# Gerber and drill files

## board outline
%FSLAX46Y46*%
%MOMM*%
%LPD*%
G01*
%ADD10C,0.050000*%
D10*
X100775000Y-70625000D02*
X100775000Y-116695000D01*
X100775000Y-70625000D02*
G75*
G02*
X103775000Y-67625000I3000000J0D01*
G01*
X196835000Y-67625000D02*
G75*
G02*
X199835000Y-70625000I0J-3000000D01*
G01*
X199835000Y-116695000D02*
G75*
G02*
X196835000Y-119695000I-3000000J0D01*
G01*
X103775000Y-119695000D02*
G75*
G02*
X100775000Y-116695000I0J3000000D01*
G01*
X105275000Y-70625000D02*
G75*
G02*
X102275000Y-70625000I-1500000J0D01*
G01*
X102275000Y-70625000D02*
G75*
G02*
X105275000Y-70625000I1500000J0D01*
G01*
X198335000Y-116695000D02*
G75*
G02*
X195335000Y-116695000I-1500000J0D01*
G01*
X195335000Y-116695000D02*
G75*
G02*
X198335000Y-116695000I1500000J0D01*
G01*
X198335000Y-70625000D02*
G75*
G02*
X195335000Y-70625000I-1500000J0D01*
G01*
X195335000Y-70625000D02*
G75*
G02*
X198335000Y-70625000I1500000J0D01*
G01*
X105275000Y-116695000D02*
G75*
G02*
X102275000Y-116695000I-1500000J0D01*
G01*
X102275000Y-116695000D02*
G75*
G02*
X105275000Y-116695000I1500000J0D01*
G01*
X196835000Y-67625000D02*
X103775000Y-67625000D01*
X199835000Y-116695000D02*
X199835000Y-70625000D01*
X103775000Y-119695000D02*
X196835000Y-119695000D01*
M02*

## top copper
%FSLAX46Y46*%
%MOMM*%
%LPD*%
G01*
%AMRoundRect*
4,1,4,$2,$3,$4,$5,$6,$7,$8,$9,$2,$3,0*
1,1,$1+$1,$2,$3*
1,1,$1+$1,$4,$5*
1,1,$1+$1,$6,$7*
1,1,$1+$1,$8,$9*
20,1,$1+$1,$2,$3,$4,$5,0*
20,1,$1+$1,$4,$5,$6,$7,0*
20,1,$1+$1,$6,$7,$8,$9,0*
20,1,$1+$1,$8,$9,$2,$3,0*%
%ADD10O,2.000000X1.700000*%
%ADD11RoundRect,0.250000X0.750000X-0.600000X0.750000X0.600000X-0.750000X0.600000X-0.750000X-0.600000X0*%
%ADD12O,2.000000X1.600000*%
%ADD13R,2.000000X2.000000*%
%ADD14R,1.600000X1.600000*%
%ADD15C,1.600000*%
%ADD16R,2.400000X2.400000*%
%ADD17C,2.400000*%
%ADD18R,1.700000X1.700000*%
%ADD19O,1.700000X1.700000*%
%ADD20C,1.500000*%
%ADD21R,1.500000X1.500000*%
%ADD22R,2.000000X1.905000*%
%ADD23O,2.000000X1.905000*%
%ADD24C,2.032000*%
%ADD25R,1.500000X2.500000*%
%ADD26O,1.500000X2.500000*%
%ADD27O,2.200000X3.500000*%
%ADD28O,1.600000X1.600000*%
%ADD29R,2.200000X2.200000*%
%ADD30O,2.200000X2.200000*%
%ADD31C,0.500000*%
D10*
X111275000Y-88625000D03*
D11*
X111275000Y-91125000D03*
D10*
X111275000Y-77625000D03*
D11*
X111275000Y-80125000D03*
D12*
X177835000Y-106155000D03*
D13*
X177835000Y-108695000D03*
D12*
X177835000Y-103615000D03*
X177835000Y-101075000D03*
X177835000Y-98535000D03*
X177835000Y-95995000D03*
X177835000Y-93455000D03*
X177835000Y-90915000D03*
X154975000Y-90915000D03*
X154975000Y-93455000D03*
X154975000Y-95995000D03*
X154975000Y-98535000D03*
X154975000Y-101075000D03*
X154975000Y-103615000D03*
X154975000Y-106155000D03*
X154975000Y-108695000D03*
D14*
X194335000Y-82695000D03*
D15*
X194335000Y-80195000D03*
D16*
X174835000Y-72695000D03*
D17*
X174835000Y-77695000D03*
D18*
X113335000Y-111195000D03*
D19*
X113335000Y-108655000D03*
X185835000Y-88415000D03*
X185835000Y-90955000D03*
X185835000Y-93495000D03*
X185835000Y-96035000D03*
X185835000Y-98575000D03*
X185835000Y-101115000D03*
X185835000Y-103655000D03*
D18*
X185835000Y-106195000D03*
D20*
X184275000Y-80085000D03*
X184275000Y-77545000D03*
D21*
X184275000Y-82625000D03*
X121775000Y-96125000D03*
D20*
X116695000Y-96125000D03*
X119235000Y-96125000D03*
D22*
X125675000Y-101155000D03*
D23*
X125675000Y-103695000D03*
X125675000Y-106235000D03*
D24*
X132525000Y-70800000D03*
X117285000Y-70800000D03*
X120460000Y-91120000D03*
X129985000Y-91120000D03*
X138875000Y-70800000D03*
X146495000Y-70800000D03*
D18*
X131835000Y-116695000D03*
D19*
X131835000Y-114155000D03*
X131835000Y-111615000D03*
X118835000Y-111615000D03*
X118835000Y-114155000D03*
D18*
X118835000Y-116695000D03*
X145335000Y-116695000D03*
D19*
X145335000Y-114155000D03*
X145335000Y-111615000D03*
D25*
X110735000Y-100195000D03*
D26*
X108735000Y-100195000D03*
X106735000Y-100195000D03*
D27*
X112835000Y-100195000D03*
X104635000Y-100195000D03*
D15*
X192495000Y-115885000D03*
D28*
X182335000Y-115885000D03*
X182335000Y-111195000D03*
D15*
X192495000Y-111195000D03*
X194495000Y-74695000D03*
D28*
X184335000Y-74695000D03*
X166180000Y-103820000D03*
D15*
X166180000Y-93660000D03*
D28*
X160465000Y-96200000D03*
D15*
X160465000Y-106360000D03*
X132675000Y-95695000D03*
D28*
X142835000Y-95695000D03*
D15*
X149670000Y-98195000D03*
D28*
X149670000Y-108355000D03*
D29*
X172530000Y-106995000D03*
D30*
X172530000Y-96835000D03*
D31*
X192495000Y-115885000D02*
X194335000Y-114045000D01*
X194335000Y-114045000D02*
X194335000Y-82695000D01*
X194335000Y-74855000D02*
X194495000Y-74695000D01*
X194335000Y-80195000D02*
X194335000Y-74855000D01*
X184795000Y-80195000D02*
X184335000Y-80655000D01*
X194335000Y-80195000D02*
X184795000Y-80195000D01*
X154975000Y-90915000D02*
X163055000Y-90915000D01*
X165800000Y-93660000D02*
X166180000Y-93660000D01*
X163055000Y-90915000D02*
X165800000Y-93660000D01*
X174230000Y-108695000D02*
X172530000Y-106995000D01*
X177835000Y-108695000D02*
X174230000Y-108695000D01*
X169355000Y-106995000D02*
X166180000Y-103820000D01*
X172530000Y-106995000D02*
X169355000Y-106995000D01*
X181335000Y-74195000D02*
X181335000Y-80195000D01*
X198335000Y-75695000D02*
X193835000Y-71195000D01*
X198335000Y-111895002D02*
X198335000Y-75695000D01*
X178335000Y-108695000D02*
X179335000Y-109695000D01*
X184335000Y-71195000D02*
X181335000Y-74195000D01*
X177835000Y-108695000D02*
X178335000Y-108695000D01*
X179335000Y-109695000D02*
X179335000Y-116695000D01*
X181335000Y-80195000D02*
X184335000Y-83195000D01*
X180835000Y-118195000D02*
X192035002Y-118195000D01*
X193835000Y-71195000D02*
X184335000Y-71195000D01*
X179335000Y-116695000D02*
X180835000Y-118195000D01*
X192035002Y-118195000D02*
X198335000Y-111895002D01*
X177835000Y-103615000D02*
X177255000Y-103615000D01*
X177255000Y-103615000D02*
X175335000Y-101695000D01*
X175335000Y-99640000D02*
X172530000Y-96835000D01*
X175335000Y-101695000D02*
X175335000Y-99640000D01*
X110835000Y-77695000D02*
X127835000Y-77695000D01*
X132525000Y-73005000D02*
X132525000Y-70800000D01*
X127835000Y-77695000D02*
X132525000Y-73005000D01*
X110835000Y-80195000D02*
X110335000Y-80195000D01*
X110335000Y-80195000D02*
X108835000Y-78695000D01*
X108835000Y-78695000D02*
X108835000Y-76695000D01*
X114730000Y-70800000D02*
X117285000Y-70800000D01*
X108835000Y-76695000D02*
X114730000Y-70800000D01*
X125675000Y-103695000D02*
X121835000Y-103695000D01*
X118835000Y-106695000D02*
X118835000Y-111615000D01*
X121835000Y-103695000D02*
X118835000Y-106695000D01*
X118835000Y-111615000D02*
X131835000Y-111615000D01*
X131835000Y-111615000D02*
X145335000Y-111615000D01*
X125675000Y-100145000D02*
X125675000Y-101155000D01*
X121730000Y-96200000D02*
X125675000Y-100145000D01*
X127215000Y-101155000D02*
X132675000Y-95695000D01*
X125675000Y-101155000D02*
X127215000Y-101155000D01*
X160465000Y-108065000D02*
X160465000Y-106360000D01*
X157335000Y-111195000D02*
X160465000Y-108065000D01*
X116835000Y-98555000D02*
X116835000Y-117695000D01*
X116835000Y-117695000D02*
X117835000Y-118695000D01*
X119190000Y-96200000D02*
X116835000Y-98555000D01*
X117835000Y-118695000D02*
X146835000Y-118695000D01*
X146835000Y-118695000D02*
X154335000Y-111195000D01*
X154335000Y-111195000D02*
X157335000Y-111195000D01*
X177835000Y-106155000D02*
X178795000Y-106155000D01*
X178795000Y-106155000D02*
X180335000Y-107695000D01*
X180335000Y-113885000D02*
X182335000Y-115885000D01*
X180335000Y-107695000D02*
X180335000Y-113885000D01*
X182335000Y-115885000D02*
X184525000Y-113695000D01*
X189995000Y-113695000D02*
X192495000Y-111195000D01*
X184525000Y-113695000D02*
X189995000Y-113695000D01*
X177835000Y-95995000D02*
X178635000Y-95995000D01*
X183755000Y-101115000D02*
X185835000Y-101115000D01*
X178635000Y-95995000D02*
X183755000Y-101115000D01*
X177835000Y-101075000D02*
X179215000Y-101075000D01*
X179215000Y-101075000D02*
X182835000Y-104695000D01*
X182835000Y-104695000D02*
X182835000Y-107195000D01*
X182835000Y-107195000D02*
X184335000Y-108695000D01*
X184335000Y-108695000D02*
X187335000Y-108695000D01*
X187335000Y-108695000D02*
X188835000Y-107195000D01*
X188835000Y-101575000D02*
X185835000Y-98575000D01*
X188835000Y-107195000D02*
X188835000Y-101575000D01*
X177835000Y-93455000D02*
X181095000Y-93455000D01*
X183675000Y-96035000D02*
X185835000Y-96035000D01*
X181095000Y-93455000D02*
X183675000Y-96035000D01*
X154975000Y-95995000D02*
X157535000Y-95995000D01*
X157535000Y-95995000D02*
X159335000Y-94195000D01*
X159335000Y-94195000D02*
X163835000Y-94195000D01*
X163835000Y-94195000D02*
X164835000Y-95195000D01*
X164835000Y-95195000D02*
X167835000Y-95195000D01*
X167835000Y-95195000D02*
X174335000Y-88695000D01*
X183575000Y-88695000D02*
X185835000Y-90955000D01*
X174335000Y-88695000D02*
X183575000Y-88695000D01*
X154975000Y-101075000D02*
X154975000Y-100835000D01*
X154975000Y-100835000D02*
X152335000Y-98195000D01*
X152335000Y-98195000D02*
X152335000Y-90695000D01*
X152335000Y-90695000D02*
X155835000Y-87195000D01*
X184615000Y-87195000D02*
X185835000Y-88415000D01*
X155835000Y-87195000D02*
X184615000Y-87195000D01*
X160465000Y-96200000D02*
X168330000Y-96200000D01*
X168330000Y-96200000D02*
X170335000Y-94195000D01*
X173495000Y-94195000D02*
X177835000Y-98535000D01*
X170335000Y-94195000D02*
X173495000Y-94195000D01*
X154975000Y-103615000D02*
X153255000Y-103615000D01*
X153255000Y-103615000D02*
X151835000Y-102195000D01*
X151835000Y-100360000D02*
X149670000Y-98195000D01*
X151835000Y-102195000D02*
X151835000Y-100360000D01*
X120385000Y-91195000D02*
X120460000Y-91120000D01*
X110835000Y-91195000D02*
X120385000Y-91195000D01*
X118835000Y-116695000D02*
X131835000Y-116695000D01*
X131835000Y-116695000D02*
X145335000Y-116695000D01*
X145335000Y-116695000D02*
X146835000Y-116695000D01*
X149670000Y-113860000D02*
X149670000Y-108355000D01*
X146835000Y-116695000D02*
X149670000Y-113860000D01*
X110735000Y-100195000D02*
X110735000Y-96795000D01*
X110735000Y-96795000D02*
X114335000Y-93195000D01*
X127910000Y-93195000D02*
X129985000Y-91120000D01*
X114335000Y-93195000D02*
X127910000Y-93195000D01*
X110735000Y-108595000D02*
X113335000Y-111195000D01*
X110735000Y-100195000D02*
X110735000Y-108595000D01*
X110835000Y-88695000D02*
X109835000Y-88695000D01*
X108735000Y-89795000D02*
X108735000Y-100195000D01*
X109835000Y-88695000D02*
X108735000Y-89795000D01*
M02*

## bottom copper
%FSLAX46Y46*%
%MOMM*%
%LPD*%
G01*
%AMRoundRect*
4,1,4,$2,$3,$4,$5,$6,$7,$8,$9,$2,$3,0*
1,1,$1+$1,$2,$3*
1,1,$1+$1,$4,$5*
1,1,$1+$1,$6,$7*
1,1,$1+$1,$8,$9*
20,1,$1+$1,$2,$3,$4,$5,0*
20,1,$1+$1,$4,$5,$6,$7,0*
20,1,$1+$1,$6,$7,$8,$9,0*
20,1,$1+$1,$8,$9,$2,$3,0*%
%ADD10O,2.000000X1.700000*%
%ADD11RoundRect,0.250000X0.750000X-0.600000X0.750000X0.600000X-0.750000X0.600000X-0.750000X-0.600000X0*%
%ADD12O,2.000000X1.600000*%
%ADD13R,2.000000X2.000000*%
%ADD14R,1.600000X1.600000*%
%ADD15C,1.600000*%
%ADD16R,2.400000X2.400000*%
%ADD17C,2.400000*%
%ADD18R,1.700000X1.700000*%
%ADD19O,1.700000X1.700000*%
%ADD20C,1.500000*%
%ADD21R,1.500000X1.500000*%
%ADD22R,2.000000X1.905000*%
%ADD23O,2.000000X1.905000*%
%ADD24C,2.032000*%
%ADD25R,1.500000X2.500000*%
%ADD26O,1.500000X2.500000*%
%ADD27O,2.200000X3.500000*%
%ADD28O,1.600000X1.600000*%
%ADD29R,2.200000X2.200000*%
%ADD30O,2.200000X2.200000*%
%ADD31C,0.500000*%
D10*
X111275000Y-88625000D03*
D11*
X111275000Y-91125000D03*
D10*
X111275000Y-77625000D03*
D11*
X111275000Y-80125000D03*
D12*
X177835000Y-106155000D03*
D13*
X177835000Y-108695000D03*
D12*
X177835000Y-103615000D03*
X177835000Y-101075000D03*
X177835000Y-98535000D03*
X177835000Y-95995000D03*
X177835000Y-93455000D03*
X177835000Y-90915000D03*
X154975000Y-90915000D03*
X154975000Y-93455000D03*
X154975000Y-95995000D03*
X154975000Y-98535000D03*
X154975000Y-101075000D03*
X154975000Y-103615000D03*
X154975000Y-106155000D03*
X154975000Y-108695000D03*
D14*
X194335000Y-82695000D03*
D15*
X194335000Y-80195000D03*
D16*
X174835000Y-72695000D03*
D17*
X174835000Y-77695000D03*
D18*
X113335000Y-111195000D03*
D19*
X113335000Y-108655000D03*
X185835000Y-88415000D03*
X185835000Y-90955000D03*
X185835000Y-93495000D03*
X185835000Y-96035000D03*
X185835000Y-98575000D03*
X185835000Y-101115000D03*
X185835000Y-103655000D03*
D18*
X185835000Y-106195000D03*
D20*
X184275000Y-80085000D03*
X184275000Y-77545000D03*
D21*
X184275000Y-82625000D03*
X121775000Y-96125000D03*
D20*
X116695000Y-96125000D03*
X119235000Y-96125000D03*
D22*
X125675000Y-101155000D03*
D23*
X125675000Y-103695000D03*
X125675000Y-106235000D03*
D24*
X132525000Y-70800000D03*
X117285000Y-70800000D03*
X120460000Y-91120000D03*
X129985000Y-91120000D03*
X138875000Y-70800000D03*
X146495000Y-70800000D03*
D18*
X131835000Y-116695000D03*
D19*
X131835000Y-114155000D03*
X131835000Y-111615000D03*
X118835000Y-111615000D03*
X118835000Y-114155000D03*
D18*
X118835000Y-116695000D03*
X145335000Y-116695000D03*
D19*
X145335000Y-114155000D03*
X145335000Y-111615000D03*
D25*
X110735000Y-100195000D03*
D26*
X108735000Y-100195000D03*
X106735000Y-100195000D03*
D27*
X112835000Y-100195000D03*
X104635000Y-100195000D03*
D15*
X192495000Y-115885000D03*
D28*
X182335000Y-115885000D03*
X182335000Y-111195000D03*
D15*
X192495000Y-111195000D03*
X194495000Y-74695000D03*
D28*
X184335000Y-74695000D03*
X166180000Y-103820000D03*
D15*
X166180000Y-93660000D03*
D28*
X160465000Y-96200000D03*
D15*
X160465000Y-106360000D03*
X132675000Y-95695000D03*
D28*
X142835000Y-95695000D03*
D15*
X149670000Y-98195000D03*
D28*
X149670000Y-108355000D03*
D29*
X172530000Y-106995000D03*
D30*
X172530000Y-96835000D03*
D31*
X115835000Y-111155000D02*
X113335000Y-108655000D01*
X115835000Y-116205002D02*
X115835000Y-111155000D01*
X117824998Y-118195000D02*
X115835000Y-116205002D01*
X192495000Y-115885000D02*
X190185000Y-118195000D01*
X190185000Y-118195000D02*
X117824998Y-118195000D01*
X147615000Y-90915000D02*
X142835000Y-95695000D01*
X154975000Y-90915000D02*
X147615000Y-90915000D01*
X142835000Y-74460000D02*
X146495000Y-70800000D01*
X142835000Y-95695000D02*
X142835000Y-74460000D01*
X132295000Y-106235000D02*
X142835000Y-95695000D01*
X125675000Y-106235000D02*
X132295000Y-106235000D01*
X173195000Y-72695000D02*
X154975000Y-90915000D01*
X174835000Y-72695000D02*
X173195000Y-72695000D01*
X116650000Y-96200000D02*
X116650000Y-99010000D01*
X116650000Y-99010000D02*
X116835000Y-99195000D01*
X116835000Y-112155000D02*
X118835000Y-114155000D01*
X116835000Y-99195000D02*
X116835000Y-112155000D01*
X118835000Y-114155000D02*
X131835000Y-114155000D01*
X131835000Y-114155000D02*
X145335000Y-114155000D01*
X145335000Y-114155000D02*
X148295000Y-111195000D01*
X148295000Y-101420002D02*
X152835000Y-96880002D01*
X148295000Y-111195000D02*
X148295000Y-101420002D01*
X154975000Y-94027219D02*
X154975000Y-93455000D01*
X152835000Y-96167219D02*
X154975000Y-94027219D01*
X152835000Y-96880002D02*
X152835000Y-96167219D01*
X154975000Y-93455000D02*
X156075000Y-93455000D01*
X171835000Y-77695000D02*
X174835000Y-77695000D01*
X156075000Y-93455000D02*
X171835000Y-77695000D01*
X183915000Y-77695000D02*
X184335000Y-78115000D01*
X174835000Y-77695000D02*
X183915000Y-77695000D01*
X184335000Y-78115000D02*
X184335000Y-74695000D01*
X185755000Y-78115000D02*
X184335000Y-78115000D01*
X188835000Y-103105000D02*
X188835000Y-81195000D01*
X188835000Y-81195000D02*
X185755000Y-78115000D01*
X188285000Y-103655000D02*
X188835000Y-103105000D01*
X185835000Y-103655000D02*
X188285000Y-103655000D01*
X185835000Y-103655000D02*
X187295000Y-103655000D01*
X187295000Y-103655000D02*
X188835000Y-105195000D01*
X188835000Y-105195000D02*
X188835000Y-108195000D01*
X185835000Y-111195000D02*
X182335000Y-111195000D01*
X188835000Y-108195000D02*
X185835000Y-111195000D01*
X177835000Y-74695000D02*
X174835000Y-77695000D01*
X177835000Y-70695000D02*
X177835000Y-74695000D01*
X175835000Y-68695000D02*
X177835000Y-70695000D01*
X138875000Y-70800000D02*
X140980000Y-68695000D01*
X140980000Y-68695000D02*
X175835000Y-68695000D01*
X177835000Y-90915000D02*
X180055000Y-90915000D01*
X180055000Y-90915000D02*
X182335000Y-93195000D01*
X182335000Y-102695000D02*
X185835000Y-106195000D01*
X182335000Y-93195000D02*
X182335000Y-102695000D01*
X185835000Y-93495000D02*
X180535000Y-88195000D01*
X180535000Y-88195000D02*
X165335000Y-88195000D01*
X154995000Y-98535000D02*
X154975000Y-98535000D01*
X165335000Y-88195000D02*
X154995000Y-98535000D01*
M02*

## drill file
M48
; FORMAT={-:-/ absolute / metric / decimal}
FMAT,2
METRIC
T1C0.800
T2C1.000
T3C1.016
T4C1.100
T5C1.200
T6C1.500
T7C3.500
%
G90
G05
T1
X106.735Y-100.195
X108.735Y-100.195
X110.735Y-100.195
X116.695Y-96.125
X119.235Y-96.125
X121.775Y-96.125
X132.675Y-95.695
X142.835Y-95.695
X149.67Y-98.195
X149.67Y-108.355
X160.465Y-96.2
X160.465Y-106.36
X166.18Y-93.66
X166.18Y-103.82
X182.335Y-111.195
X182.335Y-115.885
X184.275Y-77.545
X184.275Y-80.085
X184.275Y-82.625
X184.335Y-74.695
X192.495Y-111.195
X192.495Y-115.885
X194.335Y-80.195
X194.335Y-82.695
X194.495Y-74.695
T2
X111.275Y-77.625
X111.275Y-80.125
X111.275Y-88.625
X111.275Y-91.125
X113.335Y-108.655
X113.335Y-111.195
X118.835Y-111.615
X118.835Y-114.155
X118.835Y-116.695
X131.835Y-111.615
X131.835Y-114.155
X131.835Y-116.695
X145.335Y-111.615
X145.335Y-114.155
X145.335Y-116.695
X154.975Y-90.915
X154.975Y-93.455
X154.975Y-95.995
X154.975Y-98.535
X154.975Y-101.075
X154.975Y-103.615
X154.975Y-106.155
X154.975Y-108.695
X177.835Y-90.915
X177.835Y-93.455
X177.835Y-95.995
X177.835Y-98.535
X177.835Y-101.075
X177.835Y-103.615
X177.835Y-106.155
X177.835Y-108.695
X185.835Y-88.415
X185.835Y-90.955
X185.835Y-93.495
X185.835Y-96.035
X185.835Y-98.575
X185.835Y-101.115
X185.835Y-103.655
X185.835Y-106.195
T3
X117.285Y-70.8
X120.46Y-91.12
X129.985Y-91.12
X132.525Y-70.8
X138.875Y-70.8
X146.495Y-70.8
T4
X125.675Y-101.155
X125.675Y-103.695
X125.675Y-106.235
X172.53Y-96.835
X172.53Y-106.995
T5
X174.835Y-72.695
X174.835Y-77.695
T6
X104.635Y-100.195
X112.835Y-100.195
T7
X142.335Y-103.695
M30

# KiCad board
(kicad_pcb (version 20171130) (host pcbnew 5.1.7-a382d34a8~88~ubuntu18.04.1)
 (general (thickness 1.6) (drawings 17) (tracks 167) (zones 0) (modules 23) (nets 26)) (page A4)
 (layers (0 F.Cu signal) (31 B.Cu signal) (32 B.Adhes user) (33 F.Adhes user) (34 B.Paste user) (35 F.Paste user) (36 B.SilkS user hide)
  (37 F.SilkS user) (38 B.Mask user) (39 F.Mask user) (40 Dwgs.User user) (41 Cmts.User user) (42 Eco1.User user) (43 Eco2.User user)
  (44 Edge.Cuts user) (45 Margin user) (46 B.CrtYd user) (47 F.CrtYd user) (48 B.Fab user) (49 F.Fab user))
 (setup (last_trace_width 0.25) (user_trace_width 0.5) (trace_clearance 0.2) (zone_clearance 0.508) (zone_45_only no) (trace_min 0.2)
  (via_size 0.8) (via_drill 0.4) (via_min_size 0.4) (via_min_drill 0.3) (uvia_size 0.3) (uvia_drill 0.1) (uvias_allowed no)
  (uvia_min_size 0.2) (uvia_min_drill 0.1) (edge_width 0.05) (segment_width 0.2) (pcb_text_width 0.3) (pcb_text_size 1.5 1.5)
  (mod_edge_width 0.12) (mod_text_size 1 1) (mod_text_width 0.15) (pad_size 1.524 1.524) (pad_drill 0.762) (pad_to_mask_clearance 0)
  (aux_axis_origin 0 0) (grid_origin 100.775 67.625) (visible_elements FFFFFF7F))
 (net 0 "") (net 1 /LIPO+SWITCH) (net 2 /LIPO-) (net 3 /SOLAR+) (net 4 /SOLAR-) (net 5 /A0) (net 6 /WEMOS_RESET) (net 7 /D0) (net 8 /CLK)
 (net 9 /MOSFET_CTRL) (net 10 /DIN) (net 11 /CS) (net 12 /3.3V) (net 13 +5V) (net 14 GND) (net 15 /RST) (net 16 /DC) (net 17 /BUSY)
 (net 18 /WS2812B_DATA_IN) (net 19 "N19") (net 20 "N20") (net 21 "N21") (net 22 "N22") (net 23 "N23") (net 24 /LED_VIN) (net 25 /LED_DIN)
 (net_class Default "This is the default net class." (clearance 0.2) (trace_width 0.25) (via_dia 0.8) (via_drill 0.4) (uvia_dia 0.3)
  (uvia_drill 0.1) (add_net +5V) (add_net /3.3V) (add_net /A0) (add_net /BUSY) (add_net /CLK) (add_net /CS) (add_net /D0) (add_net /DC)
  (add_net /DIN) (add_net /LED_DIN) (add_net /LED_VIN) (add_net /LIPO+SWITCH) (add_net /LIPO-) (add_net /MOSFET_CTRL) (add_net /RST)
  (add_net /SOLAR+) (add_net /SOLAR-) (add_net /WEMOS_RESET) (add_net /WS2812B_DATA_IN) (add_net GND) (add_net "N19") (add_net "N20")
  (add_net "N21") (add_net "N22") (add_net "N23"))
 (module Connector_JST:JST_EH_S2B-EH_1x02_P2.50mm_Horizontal (layer F.Cu) (at 111.275 91.125 90)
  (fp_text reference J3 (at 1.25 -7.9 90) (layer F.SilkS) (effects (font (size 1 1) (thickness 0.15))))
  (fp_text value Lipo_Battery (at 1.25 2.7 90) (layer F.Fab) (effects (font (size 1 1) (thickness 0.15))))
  (pad 2 thru_hole oval (at 2.5 0 90) (size 1.7 2) (drill 1) (layers *.Cu *.Mask) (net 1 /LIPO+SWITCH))
  (pad 1 thru_hole roundrect (at 0 0 90) (size 1.7 2) (drill 1) (layers *.Cu *.Mask) (roundrect_rratio 0.147059) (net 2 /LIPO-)))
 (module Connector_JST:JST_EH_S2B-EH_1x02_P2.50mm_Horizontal (layer F.Cu) (at 111.275 80.125 90)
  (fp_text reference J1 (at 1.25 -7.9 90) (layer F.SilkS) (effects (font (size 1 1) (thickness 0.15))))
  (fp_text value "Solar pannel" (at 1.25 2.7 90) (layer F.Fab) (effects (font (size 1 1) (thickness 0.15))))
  (pad 2 thru_hole oval (at 2.5 0 90) (size 1.7 2) (drill 1) (layers *.Cu *.Mask) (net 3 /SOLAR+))
  (pad 1 thru_hole roundrect (at 0 0 90) (size 1.7 2) (drill 1) (layers *.Cu *.Mask) (roundrect_rratio 0.147059) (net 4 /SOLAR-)))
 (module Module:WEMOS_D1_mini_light (layer F.Cu) (at 177.835 108.695 180)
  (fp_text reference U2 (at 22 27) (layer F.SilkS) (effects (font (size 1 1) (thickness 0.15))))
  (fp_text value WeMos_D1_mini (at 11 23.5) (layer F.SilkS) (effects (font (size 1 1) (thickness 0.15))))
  (pad 2 thru_hole oval (at 0 2.54 180) (size 2 1.6) (drill 1) (layers *.Cu *.Mask) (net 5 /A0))
  (pad 1 thru_hole rect (at 0 0 180) (size 2 2) (drill 1) (layers *.Cu *.Mask) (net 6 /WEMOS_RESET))
  (pad 3 thru_hole oval (at 0 5.08 180) (size 2 1.6) (drill 1) (layers *.Cu *.Mask) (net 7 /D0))
  (pad 4 thru_hole oval (at 0 7.62 180) (size 2 1.6) (drill 1) (layers *.Cu *.Mask) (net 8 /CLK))
  (pad 5 thru_hole oval (at 0 10.16 180) (size 2 1.6) (drill 1) (layers *.Cu *.Mask) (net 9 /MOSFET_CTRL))
  (pad 6 thru_hole oval (at 0 12.7 180) (size 2 1.6) (drill 1) (layers *.Cu *.Mask) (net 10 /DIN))
  (pad 7 thru_hole oval (at 0 15.24 180) (size 2 1.6) (drill 1) (layers *.Cu *.Mask) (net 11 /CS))
  (pad 8 thru_hole oval (at 0 17.78 180) (size 2 1.6) (drill 1) (layers *.Cu *.Mask) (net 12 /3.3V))
  (pad 9 thru_hole oval (at 22.86 17.78 180) (size 2 1.6) (drill 1) (layers *.Cu *.Mask) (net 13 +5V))
  (pad 10 thru_hole oval (at 22.86 15.24 180) (size 2 1.6) (drill 1) (layers *.Cu *.Mask) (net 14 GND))
  (pad 11 thru_hole oval (at 22.86 12.7 180) (size 2 1.6) (drill 1) (layers *.Cu *.Mask) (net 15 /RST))
  (pad 12 thru_hole oval (at 22.86 10.16 180) (size 2 1.6) (drill 1) (layers *.Cu *.Mask) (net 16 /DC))
  (pad 13 thru_hole oval (at 22.86 7.62 180) (size 2 1.6) (drill 1) (layers *.Cu *.Mask) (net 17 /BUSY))
  (pad 14 thru_hole oval (at 22.86 5.08 180) (size 2 1.6) (drill 1) (layers *.Cu *.Mask) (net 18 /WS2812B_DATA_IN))
  (pad 15 thru_hole oval (at 22.86 2.54 180) (size 2 1.6) (drill 1) (layers *.Cu *.Mask))
  (pad 16 thru_hole oval (at 22.86 0 180) (size 2 1.6) (drill 1) (layers *.Cu *.Mask)))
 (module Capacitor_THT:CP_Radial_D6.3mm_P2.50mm (layer F.Cu) (at 194.335 82.695 90)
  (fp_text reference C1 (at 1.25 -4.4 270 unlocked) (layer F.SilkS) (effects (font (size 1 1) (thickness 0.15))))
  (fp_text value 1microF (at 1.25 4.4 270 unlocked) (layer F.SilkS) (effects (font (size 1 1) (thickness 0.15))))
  (pad 1 thru_hole rect (at 0 0 90) (size 1.6 1.6) (drill 0.8) (layers *.Cu *.Mask) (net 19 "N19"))
  (pad 2 thru_hole circle (at 2.5 0 90) (size 1.6 1.6) (drill 0.8) (layers *.Cu *.Mask) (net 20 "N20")))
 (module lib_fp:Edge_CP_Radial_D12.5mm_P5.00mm (layer F.Cu) (at 174.835 75.195 270)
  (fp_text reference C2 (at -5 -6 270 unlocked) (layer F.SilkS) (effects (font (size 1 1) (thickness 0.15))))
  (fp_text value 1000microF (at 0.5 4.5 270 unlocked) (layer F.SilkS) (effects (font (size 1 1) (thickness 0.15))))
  (pad 1 thru_hole rect (at -2.5 0 270) (size 2.4 2.4) (drill 1.2) (layers *.Cu *.Mask) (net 13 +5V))
  (pad 2 thru_hole circle (at 2.5 0 270) (size 2.4 2.4) (drill 1.2) (layers *.Cu *.Mask) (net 14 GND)))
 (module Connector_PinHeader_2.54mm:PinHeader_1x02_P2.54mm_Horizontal (layer F.Cu) (at 113.335 111.195 180)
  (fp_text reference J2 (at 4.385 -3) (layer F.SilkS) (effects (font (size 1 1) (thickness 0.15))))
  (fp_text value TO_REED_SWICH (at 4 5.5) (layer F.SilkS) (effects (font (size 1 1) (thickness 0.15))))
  (pad 1 thru_hole rect (at 0 0 180) (size 1.7 1.7) (drill 1) (layers *.Cu *.Mask) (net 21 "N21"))
  (pad 2 thru_hole oval (at 0 2.54 180) (size 1.7 1.7) (drill 1) (layers *.Cu *.Mask) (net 19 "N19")))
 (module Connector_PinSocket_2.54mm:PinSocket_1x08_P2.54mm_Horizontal (layer F.Cu) (at 185.835 106.195 180)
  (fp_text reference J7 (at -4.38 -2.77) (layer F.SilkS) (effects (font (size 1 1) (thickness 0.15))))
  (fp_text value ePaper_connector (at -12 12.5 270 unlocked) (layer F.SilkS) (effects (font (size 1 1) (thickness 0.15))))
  (pad 8 thru_hole oval (at 0 17.78 180) (size 1.7 1.7) (drill 1) (layers *.Cu *.Mask) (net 17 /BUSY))
  (pad 7 thru_hole oval (at 0 15.24 180) (size 1.7 1.7) (drill 1) (layers *.Cu *.Mask) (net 15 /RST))
  (pad 6 thru_hole oval (at 0 12.7 180) (size 1.7 1.7) (drill 1) (layers *.Cu *.Mask) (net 16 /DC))
  (pad 5 thru_hole oval (at 0 10.16 180) (size 1.7 1.7) (drill 1) (layers *.Cu *.Mask) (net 11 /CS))
  (pad 4 thru_hole oval (at 0 7.62 180) (size 1.7 1.7) (drill 1) (layers *.Cu *.Mask) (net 8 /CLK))
  (pad 3 thru_hole oval (at 0 5.08 180) (size 1.7 1.7) (drill 1) (layers *.Cu *.Mask) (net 10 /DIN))
  (pad 2 thru_hole oval (at 0 2.54 180) (size 1.7 1.7) (drill 1) (layers *.Cu *.Mask) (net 14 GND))
  (pad 1 thru_hole rect (at 0 0 180) (size 1.7 1.7) (drill 1) (layers *.Cu *.Mask) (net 12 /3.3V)))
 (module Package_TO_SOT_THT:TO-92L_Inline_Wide (layer F.Cu) (at 184.275 82.625 90)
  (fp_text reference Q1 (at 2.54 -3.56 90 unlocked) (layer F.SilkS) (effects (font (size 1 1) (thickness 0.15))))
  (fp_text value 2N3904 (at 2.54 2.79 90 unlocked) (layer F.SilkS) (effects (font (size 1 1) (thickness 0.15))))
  (pad 2 thru_hole circle (at 2.54 0 90) (size 1.5 1.5) (drill 0.8) (layers *.Cu *.Mask) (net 20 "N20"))
  (pad 3 thru_hole circle (at 5.08 0 90) (size 1.5 1.5) (drill 0.8) (layers *.Cu *.Mask) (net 14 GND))
  (pad 1 thru_hole rect (at 0 0 90) (size 1.5 1.5) (drill 0.8) (layers *.Cu *.Mask) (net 6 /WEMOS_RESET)))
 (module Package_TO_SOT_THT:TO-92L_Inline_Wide (layer F.Cu) (at 121.775 96.125 180)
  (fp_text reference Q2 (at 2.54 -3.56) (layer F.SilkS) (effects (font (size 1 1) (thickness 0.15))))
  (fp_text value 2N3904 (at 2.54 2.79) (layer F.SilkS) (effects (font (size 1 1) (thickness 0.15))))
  (pad 1 thru_hole rect (at 0 0 180) (size 1.5 1.5) (drill 0.8) (layers *.Cu *.Mask) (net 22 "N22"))
  (pad 3 thru_hole circle (at 5.08 0 180) (size 1.5 1.5) (drill 0.8) (layers *.Cu *.Mask) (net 14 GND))
  (pad 2 thru_hole circle (at 2.54 0 180) (size 1.5 1.5) (drill 0.8) (layers *.Cu *.Mask) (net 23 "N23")))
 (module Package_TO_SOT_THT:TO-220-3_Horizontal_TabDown (layer F.Cu) (at 125.675 101.155 270)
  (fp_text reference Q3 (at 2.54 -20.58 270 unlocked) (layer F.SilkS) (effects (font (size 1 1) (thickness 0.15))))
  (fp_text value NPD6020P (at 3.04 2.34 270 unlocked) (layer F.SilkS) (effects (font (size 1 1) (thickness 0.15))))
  (pad "" np_thru_hole oval (at 2.54 -16.66 270) (size 3.5 3.5) (drill 3.5) (layers *.Cu *.Mask))
  (pad 1 thru_hole rect (at 0 0 270) (size 1.905 2) (drill 1.1) (layers *.Cu *.Mask) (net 22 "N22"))
  (pad 2 thru_hole oval (at 2.54 0 270) (size 1.905 2) (drill 1.1) (layers *.Cu *.Mask) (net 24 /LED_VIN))
  (pad 3 thru_hole oval (at 5.08 0 270) (size 1.905 2) (drill 1.1) (layers *.Cu *.Mask) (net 13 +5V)))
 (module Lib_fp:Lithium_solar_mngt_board (layer F.Cu) (at 135.065 66.99)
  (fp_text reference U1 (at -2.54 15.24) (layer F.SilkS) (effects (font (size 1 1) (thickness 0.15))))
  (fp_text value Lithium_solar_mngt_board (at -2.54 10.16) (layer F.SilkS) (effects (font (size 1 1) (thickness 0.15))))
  (pad 1 thru_hole circle (at -2.54 3.81) (size 2.032 2.032) (drill 1.016) (layers *.Cu *.Mask) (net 3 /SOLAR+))
  (pad 2 thru_hole circle (at -17.78 3.81) (size 2.032 2.032) (drill 1.016) (layers *.Cu *.Mask) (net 4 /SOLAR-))
  (pad 4 thru_hole circle (at -14.605 24.13) (size 2.032 2.032) (drill 1.016) (layers *.Cu *.Mask) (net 2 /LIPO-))
  (pad 3 thru_hole circle (at -5.08 24.13) (size 2.032 2.032) (drill 1.016) (layers *.Cu *.Mask) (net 21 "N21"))
  (pad 6 thru_hole circle (at 3.81 3.81) (size 2.032 2.032) (drill 1.016) (layers *.Cu *.Mask) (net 14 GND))
  (pad 5 thru_hole circle (at 11.43 3.81) (size 2.032 2.032) (drill 1.016) (layers *.Cu *.Mask) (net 13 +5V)))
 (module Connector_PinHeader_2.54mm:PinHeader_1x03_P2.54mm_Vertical (layer F.Cu) (at 131.835 116.695 180)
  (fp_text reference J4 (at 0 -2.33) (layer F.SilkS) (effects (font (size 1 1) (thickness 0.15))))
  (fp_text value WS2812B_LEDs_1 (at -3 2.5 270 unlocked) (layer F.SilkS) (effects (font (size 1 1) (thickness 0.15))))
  (pad 1 thru_hole rect (at 0 0 180) (size 1.7 1.7) (drill 1) (layers *.Cu *.Mask) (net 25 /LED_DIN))
  (pad 2 thru_hole oval (at 0 2.54 180) (size 1.7 1.7) (drill 1) (layers *.Cu *.Mask) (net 14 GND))
  (pad 3 thru_hole oval (at 0 5.08 180) (size 1.7 1.7) (drill 1) (layers *.Cu *.Mask) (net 24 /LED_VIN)))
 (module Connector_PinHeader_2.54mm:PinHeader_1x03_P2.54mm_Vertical (layer F.Cu) (at 118.835 116.695 180)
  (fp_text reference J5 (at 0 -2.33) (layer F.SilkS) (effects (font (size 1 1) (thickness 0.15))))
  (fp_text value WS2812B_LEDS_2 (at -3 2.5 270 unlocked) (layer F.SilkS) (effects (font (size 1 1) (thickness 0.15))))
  (pad 3 thru_hole oval (at 0 5.08 180) (size 1.7 1.7) (drill 1) (layers *.Cu *.Mask) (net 24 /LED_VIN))
  (pad 2 thru_hole oval (at 0 2.54 180) (size 1.7 1.7) (drill 1) (layers *.Cu *.Mask) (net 14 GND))
  (pad 1 thru_hole rect (at 0 0 180) (size 1.7 1.7) (drill 1) (layers *.Cu *.Mask) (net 25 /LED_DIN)))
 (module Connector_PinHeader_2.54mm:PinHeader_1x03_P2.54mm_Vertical (layer F.Cu) (at 145.335 116.695 180)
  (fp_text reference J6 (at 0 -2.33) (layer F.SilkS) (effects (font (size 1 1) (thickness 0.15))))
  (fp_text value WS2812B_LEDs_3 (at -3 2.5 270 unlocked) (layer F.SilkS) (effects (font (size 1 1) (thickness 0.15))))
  (pad 1 thru_hole rect (at 0 0 180) (size 1.7 1.7) (drill 1) (layers *.Cu *.Mask) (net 25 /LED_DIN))
  (pad 2 thru_hole oval (at 0 2.54 180) (size 1.7 1.7) (drill 1) (layers *.Cu *.Mask) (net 14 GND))
  (pad 3 thru_hole oval (at 0 5.08 180) (size 1.7 1.7) (drill 1) (layers *.Cu *.Mask) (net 24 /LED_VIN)))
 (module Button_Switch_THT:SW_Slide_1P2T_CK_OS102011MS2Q (layer F.Cu) (at 110.735 100.195 180)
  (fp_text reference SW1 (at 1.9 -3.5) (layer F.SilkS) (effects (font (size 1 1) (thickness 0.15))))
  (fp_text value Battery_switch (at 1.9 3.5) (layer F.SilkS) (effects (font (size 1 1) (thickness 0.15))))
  (pad 1 thru_hole rect (at 0 0 180) (size 1.5 2.5) (drill 0.8) (layers *.Cu *.Mask) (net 21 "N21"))
  (pad 2 thru_hole oval (at 2 0 180) (size 1.5 2.5) (drill 0.8) (layers *.Cu *.Mask) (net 1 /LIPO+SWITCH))
  (pad 3 thru_hole oval (at 4 0 180) (size 1.5 2.5) (drill 0.8) (layers *.Cu *.Mask))
  (pad "" thru_hole oval (at -2.1 0 180) (size 2.2 3.5) (drill 1.5) (layers *.Cu *.Mask))
  (pad "" thru_hole oval (at 6.1 0 180) (size 2.2 3.5) (drill 1.5) (layers *.Cu *.Mask)))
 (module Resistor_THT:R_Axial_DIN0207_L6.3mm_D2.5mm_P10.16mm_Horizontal (layer F.Cu) (at 192.495 115.885 180)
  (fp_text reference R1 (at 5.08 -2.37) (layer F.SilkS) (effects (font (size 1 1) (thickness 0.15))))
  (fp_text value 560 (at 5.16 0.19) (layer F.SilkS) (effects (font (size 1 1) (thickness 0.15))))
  (pad 1 thru_hole circle (at 0 0 180) (size 1.6 1.6) (drill 0.8) (layers *.Cu *.Mask) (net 19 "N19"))
  (pad 2 thru_hole oval (at 10.16 0 180) (size 1.6 1.6) (drill 0.8) (layers *.Cu *.Mask) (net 5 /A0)))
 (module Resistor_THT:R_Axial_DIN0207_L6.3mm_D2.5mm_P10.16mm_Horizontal (layer F.Cu) (at 192.495 111.195 180)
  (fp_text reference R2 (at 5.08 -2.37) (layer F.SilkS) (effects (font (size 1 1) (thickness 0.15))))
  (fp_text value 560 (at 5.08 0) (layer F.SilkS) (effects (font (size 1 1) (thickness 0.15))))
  (pad 2 thru_hole oval (at 10.16 0 180) (size 1.6 1.6) (drill 0.8) (layers *.Cu *.Mask) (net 14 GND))
  (pad 1 thru_hole circle (at 0 0 180) (size 1.6 1.6) (drill 0.8) (layers *.Cu *.Mask) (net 5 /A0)))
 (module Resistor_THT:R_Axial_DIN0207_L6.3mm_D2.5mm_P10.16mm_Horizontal (layer F.Cu) (at 194.495 74.695 180)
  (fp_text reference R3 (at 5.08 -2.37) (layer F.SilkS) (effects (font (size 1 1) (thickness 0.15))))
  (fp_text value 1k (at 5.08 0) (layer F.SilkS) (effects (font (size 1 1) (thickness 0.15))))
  (pad 1 thru_hole circle (at 0 0 180) (size 1.6 1.6) (drill 0.8) (layers *.Cu *.Mask) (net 20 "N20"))
  (pad 2 thru_hole oval (at 10.16 0 180) (size 1.6 1.6) (drill 0.8) (layers *.Cu *.Mask) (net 14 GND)))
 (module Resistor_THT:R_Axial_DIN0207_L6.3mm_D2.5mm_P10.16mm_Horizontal (layer F.Cu) (at 166.18 93.66 270)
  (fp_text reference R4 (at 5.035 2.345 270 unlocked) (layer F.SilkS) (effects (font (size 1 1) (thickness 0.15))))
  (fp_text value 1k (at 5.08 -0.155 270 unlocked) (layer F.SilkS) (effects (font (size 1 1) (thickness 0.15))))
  (pad 2 thru_hole oval (at 10.16 0 270) (size 1.6 1.6) (drill 0.8) (layers *.Cu *.Mask) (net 6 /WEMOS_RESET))
  (pad 1 thru_hole circle (at 0 0 270) (size 1.6 1.6) (drill 0.8) (layers *.Cu *.Mask) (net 13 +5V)))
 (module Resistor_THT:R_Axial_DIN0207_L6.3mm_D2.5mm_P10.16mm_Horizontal (layer F.Cu) (at 160.465 106.36 90)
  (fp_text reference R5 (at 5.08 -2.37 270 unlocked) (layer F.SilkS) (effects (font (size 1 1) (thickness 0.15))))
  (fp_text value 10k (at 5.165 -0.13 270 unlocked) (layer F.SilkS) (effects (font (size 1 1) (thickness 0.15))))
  (pad 2 thru_hole oval (at 10.16 0 90) (size 1.6 1.6) (drill 0.8) (layers *.Cu *.Mask) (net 9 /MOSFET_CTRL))
  (pad 1 thru_hole circle (at 0 0 90) (size 1.6 1.6) (drill 0.8) (layers *.Cu *.Mask) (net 23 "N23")))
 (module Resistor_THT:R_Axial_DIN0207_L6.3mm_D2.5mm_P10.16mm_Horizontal (layer F.Cu) (at 132.675 95.695)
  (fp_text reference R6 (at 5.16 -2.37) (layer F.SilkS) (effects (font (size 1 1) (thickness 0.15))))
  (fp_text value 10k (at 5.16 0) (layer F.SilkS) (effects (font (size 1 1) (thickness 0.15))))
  (pad 1 thru_hole circle (at 0 0) (size 1.6 1.6) (drill 0.8) (layers *.Cu *.Mask) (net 22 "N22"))
  (pad 2 thru_hole oval (at 10.16 0) (size 1.6 1.6) (drill 0.8) (layers *.Cu *.Mask) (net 13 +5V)))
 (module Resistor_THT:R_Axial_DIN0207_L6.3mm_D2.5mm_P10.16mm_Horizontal (layer F.Cu) (at 149.67 98.195 270)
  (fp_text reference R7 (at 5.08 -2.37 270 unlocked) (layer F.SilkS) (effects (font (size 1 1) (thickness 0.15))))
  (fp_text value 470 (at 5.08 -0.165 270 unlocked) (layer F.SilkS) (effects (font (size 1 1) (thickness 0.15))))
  (pad 1 thru_hole circle (at 0 0 270) (size 1.6 1.6) (drill 0.8) (layers *.Cu *.Mask) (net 18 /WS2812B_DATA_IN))
  (pad 2 thru_hole oval (at 10.16 0 270) (size 1.6 1.6) (drill 0.8) (layers *.Cu *.Mask) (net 25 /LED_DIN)))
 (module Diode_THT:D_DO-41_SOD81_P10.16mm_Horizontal (layer F.Cu) (at 172.53 106.995 90)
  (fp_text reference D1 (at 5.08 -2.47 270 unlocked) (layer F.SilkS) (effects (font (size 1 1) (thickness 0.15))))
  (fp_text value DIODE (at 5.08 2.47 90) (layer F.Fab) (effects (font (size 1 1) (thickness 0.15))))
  (pad 1 thru_hole rect (at 0 0 90) (size 2.2 2.2) (drill 1.1) (layers *.Cu *.Mask) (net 6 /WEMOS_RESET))
  (pad 2 thru_hole oval (at 10.16 0 90) (size 2.2 2.2) (drill 1.1) (layers *.Cu *.Mask) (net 7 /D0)))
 (gr_line (start 100.775 70.625) (end 100.775 116.695) (layer Edge.Cuts) (width 0.05))
 (gr_arc (start 103.775 70.625) (end 103.775 67.625) (angle -90) (layer Edge.Cuts) (width 0.05))
 (gr_arc (start 196.835 70.625) (end 199.835 70.625) (angle -90) (layer Edge.Cuts) (width 0.05))
 (gr_arc (start 196.835 116.695) (end 196.835 119.695) (angle -90) (layer Edge.Cuts) (width 0.05))
 (gr_arc (start 103.775 116.695) (end 100.775 116.695) (angle -90) (layer Edge.Cuts) (width 0.05))
 (gr_circle (center 103.775 70.625) (end 102.275 70.625) (layer Edge.Cuts) (width 0.05))
 (gr_circle (center 196.835 116.695) (end 198.335 116.695) (layer Edge.Cuts) (width 0.05))
 (gr_circle (center 196.835 70.625) (end 198.335 70.625) (layer Edge.Cuts) (width 0.05))
 (gr_circle (center 103.775 116.695) (end 102.275 116.695) (layer Edge.Cuts) (width 0.05))
 (gr_line (start 196.835 67.625) (end 103.775 67.625) (layer Edge.Cuts) (width 0.05))
 (gr_line (start 199.835 116.695) (end 199.835 70.625) (layer Edge.Cuts) (width 0.05))
 (gr_line (start 103.775 119.695) (end 196.835 119.695) (layer Edge.Cuts) (width 0.05))
 (segment (start 192.495 115.885) (end 194.335 114.045) (width 0.5) (layer F.Cu) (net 19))
 (segment (start 194.335 114.045) (end 194.335 82.695) (width 0.5) (layer F.Cu) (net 19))
 (segment (start 115.835 111.155) (end 113.335 108.655) (width 0.5) (layer B.Cu) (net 19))
 (segment (start 115.835 116.205002) (end 115.835 111.155) (width 0.5) (layer B.Cu) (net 19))
 (segment (start 117.824998 118.195) (end 115.835 116.205002) (width 0.5) (layer B.Cu) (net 19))
 (segment (start 192.495 115.885) (end 190.185 118.195) (width 0.5) (layer B.Cu) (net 19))
 (segment (start 190.185 118.195) (end 117.824998 118.195) (width 0.5) (layer B.Cu) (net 19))
 (segment (start 194.335 74.855) (end 194.495 74.695) (width 0.5) (layer F.Cu) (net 20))
 (segment (start 194.335 80.195) (end 194.335 74.855) (width 0.5) (layer F.Cu) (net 20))
 (segment (start 184.795 80.195) (end 184.335 80.655) (width 0.5) (layer F.Cu) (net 20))
 (segment (start 194.335 80.195) (end 184.795 80.195) (width 0.5) (layer F.Cu) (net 20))
 (segment (start 154.975 90.915) (end 163.055 90.915) (width 0.5) (layer F.Cu) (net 13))
 (segment (start 165.8 93.66) (end 166.18 93.66) (width 0.5) (layer F.Cu) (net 13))
 (segment (start 163.055 90.915) (end 165.8 93.66) (width 0.5) (layer F.Cu) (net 13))
 (segment (start 147.615 90.915) (end 142.835 95.695) (width 0.5) (layer B.Cu) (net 13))
 (segment (start 154.975 90.915) (end 147.615 90.915) (width 0.5) (layer B.Cu) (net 13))
 (segment (start 142.835 74.46) (end 146.495 70.8) (width 0.5) (layer B.Cu) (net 13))
 (segment (start 142.835 95.695) (end 142.835 74.46) (width 0.5) (layer B.Cu) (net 13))
 (segment (start 132.295 106.235) (end 142.835 95.695) (width 0.5) (layer B.Cu) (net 13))
 (segment (start 125.675 106.235) (end 132.295 106.235) (width 0.5) (layer B.Cu) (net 13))
 (segment (start 173.195 72.695) (end 154.975 90.915) (width 0.5) (layer B.Cu) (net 13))
 (segment (start 174.835 72.695) (end 173.195 72.695) (width 0.5) (layer B.Cu) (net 13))
 (segment (start 116.65 96.2) (end 116.65 99.01) (width 0.5) (layer B.Cu) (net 14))
 (segment (start 116.65 99.01) (end 116.835 99.195) (width 0.5) (layer B.Cu) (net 14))
 (segment (start 116.835 112.155) (end 118.835 114.155) (width 0.5) (layer B.Cu) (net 14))
 (segment (start 116.835 99.195) (end 116.835 112.155) (width 0.5) (layer B.Cu) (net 14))
 (segment (start 118.835 114.155) (end 131.835 114.155) (width 0.5) (layer B.Cu) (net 14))
 (segment (start 131.835 114.155) (end 145.335 114.155) (width 0.5) (layer B.Cu) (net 14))
 (segment (start 145.335 114.155) (end 148.295 111.195) (width 0.5) (layer B.Cu) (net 14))
 (segment (start 148.295 101.420002) (end 152.835 96.880002) (width 0.5) (layer B.Cu) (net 14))
 (segment (start 148.295 111.195) (end 148.295 101.420002) (width 0.5) (layer B.Cu) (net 14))
 (segment (start 154.975 94.027219) (end 154.975 93.455) (width 0.5) (layer B.Cu) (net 14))
 (segment (start 152.835 96.167219) (end 154.975 94.027219) (width 0.5) (layer B.Cu) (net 14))
 (segment (start 152.835 96.880002) (end 152.835 96.167219) (width 0.5) (layer B.Cu) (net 14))
 (segment (start 154.975 93.455) (end 156.075 93.455) (width 0.5) (layer B.Cu) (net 14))
 (segment (start 171.835 77.695) (end 174.835 77.695) (width 0.5) (layer B.Cu) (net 14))
 (segment (start 156.075 93.455) (end 171.835 77.695) (width 0.5) (layer B.Cu) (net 14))
 (segment (start 183.915 77.695) (end 184.335 78.115) (width 0.5) (layer B.Cu) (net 14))
 (segment (start 174.835 77.695) (end 183.915 77.695) (width 0.5) (layer B.Cu) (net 14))
 (segment (start 184.335 78.115) (end 184.335 74.695) (width 0.5) (layer B.Cu) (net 14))
 (segment (start 185.755 78.115) (end 184.335 78.115) (width 0.5) (layer B.Cu) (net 14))
 (segment (start 188.835 103.105) (end 188.835 81.195) (width 0.5) (layer B.Cu) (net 14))
 (segment (start 188.835 81.195) (end 185.755 78.115) (width 0.5) (layer B.Cu) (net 14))
 (segment (start 188.285 103.655) (end 188.835 103.105) (width 0.5) (layer B.Cu) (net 14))
 (segment (start 185.835 103.655) (end 188.285 103.655) (width 0.5) (layer B.Cu) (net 14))
 (segment (start 185.835 103.655) (end 187.295 103.655) (width 0.5) (layer B.Cu) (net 14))
 (segment (start 187.295 103.655) (end 188.835 105.195) (width 0.5) (layer B.Cu) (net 14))
 (segment (start 188.835 105.195) (end 188.835 108.195) (width 0.5) (layer B.Cu) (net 14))
 (segment (start 185.835 111.195) (end 182.335 111.195) (width 0.5) (layer B.Cu) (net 14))
 (segment (start 188.835 108.195) (end 185.835 111.195) (width 0.5) (layer B.Cu) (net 14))
 (segment (start 177.835 74.695) (end 174.835 77.695) (width 0.5) (layer B.Cu) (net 14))
 (segment (start 177.835 70.695) (end 177.835 74.695) (width 0.5) (layer B.Cu) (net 14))
 (segment (start 175.835 68.695) (end 177.835 70.695) (width 0.5) (layer B.Cu) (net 14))
 (segment (start 138.875 70.8) (end 140.98 68.695) (width 0.5) (layer B.Cu) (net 14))
 (segment (start 140.98 68.695) (end 175.835 68.695) (width 0.5) (layer B.Cu) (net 14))
 (segment (start 174.23 108.695) (end 172.53 106.995) (width 0.5) (layer F.Cu) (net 6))
 (segment (start 177.835 108.695) (end 174.23 108.695) (width 0.5) (layer F.Cu) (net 6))
 (segment (start 169.355 106.995) (end 166.18 103.82) (width 0.5) (layer F.Cu) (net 6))
 (segment (start 172.53 106.995) (end 169.355 106.995) (width 0.5) (layer F.Cu) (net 6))
 (segment (start 181.335 74.195) (end 181.335 80.195) (width 0.5) (layer F.Cu) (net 6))
 (segment (start 198.335 75.695) (end 193.835 71.195) (width 0.5) (layer F.Cu) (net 6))
 (segment (start 198.335 111.895002) (end 198.335 75.695) (width 0.5) (layer F.Cu) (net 6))
 (segment (start 178.335 108.695) (end 179.335 109.695) (width 0.5) (layer F.Cu) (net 6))
 (segment (start 184.335 71.195) (end 181.335 74.195) (width 0.5) (layer F.Cu) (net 6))
 (segment (start 177.835 108.695) (end 178.335 108.695) (width 0.5) (layer F.Cu) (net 6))
 (segment (start 179.335 109.695) (end 179.335 116.695) (width 0.5) (layer F.Cu) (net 6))
 (segment (start 181.335 80.195) (end 184.335 83.195) (width 0.5) (layer F.Cu) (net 6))
 (segment (start 180.835 118.195) (end 192.035002 118.195) (width 0.5) (layer F.Cu) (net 6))
 (segment (start 193.835 71.195) (end 184.335 71.195) (width 0.5) (layer F.Cu) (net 6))
 (segment (start 179.335 116.695) (end 180.835 118.195) (width 0.5) (layer F.Cu) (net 6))
 (segment (start 192.035002 118.195) (end 198.335 111.895002) (width 0.5) (layer F.Cu) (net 6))
 (segment (start 177.835 103.615) (end 177.255 103.615) (width 0.5) (layer F.Cu) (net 7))
 (segment (start 177.255 103.615) (end 175.335 101.695) (width 0.5) (layer F.Cu) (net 7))
 (segment (start 175.335 99.64) (end 172.53 96.835) (width 0.5) (layer F.Cu) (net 7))
 (segment (start 175.335 101.695) (end 175.335 99.64) (width 0.5) (layer F.Cu) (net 7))
 (segment (start 110.835 77.695) (end 127.835 77.695) (width 0.5) (layer F.Cu) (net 3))
 (segment (start 132.525 73.005) (end 132.525 70.8) (width 0.5) (layer F.Cu) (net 3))
 (segment (start 127.835 77.695) (end 132.525 73.005) (width 0.5) (layer F.Cu) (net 3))
 (segment (start 110.835 80.195) (end 110.335 80.195) (width 0.5) (layer F.Cu) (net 4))
 (segment (start 110.335 80.195) (end 108.835 78.695) (width 0.5) (layer F.Cu) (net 4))
 (segment (start 108.835 78.695) (end 108.835 76.695) (width 0.5) (layer F.Cu) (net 4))
 (segment (start 114.73 70.8) (end 117.285 70.8) (width 0.5) (layer F.Cu) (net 4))
 (segment (start 108.835 76.695) (end 114.73 70.8) (width 0.5) (layer F.Cu) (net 4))
 (segment (start 125.675 103.695) (end 121.835 103.695) (width 0.5) (layer F.Cu) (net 24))
 (segment (start 118.835 106.695) (end 118.835 111.615) (width 0.5) (layer F.Cu) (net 24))
 (segment (start 121.835 103.695) (end 118.835 106.695) (width 0.5) (layer F.Cu) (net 24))
 (segment (start 118.835 111.615) (end 131.835 111.615) (width 0.5) (layer F.Cu) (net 24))
 (segment (start 131.835 111.615) (end 145.335 111.615) (width 0.5) (layer F.Cu) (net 24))
 (segment (start 177.835 90.915) (end 180.055 90.915) (width 0.5) (layer B.Cu) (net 12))
 (segment (start 180.055 90.915) (end 182.335 93.195) (width 0.5) (layer B.Cu) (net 12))
 (segment (start 182.335 102.695) (end 185.835 106.195) (width 0.5) (layer B.Cu) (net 12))
 (segment (start 182.335 93.195) (end 182.335 102.695) (width 0.5) (layer B.Cu) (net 12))
 (segment (start 125.675 100.145) (end 125.675 101.155) (width 0.5) (layer F.Cu) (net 22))
 (segment (start 121.73 96.2) (end 125.675 100.145) (width 0.5) (layer F.Cu) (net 22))
 (segment (start 127.215 101.155) (end 132.675 95.695) (width 0.5) (layer F.Cu) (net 22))
 (segment (start 125.675 101.155) (end 127.215 101.155) (width 0.5) (layer F.Cu) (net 22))
 (segment (start 160.465 108.065) (end 160.465 106.36) (width 0.5) (layer F.Cu) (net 23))
 (segment (start 157.335 111.195) (end 160.465 108.065) (width 0.5) (layer F.Cu) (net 23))
 (segment (start 116.835 98.555) (end 116.835 117.695) (width 0.5) (layer F.Cu) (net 23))
 (segment (start 116.835 117.695) (end 117.835 118.695) (width 0.5) (layer F.Cu) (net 23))
 (segment (start 119.19 96.2) (end 116.835 98.555) (width 0.5) (layer F.Cu) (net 23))
 (segment (start 117.835 118.695) (end 146.835 118.695) (width 0.5) (layer F.Cu) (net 23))
 (segment (start 146.835 118.695) (end 154.335 111.195) (width 0.5) (layer F.Cu) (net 23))
 (segment (start 154.335 111.195) (end 157.335 111.195) (width 0.5) (layer F.Cu) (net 23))
 (segment (start 177.835 106.155) (end 178.795 106.155) (width 0.5) (layer F.Cu) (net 5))
 (segment (start 178.795 106.155) (end 180.335 107.695) (width 0.5) (layer F.Cu) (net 5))
 (segment (start 180.335 113.885) (end 182.335 115.885) (width 0.5) (layer F.Cu) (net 5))
 (segment (start 180.335 107.695) (end 180.335 113.885) (width 0.5) (layer F.Cu) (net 5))
 (segment (start 182.335 115.885) (end 184.525 113.695) (width 0.5) (layer F.Cu) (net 5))
 (segment (start 189.995 113.695) (end 192.495 111.195) (width 0.5) (layer F.Cu) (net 5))
 (segment (start 184.525 113.695) (end 189.995 113.695) (width 0.5) (layer F.Cu) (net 5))
 (segment (start 177.835 95.995) (end 178.635 95.995) (width 0.5) (layer F.Cu) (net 10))
 (segment (start 183.755 101.115) (end 185.835 101.115) (width 0.5) (layer F.Cu) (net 10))
 (segment (start 178.635 95.995) (end 183.755 101.115) (width 0.5) (layer F.Cu) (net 10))
 (segment (start 177.835 101.075) (end 179.215 101.075) (width 0.5) (layer F.Cu) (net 8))
 (segment (start 179.215 101.075) (end 182.835 104.695) (width 0.5) (layer F.Cu) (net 8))
 (segment (start 182.835 104.695) (end 182.835 107.195) (width 0.5) (layer F.Cu) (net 8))
 (segment (start 182.835 107.195) (end 184.335 108.695) (width 0.5) (layer F.Cu) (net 8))
 (segment (start 184.335 108.695) (end 187.335 108.695) (width 0.5) (layer F.Cu) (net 8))
 (segment (start 187.335 108.695) (end 188.835 107.195) (width 0.5) (layer F.Cu) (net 8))
 (segment (start 188.835 101.575) (end 185.835 98.575) (width 0.5) (layer F.Cu) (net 8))
 (segment (start 188.835 107.195) (end 188.835 101.575) (width 0.5) (layer F.Cu) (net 8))
 (segment (start 177.835 93.455) (end 181.095 93.455) (width 0.5) (layer F.Cu) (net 11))
 (segment (start 183.675 96.035) (end 185.835 96.035) (width 0.5) (layer F.Cu) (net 11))
 (segment (start 181.095 93.455) (end 183.675 96.035) (width 0.5) (layer F.Cu) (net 11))
 (segment (start 185.835 93.495) (end 180.535 88.195) (width 0.5) (layer B.Cu) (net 16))
 (segment (start 180.535 88.195) (end 165.335 88.195) (width 0.5) (layer B.Cu) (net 16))
 (segment (start 154.995 98.535) (end 154.975 98.535) (width 0.5) (layer B.Cu) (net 16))
 (segment (start 165.335 88.195) (end 154.995 98.535) (width 0.5) (layer B.Cu) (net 16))
 (segment (start 154.975 95.995) (end 157.535 95.995) (width 0.5) (layer F.Cu) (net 15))
 (segment (start 157.535 95.995) (end 159.335 94.195) (width 0.5) (layer F.Cu) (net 15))
 (segment (start 159.335 94.195) (end 163.835 94.195) (width 0.5) (layer F.Cu) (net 15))
 (segment (start 163.835 94.195) (end 164.835 95.195) (width 0.5) (layer F.Cu) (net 15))
 (segment (start 164.835 95.195) (end 167.835 95.195) (width 0.5) (layer F.Cu) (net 15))
 (segment (start 167.835 95.195) (end 174.335 88.695) (width 0.5) (layer F.Cu) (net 15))
 (segment (start 183.575 88.695) (end 185.835 90.955) (width 0.5) (layer F.Cu) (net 15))
 (segment (start 174.335 88.695) (end 183.575 88.695) (width 0.5) (layer F.Cu) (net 15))
 (segment (start 154.975 101.075) (end 154.975 100.835) (width 0.5) (layer F.Cu) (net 17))
 (segment (start 154.975 100.835) (end 152.335 98.195) (width 0.5) (layer F.Cu) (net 17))
 (segment (start 152.335 98.195) (end 152.335 90.695) (width 0.5) (layer F.Cu) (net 17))
 (segment (start 152.335 90.695) (end 155.835 87.195) (width 0.5) (layer F.Cu) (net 17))
 (segment (start 184.615 87.195) (end 185.835 88.415) (width 0.5) (layer F.Cu) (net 17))
 (segment (start 155.835 87.195) (end 184.615 87.195) (width 0.5) (layer F.Cu) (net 17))
 (segment (start 160.465 96.2) (end 168.33 96.2) (width 0.5) (layer F.Cu) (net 9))
 (segment (start 168.33 96.2) (end 170.335 94.195) (width 0.5) (layer F.Cu) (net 9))
 (segment (start 173.495 94.195) (end 177.835 98.535) (width 0.5) (layer F.Cu) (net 9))
 (segment (start 170.335 94.195) (end 173.495 94.195) (width 0.5) (layer F.Cu) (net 9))
 (segment (start 154.975 103.615) (end 153.255 103.615) (width 0.5) (layer F.Cu) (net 18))
 (segment (start 153.255 103.615) (end 151.835 102.195) (width 0.5) (layer F.Cu) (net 18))
 (segment (start 151.835 100.36) (end 149.67 98.195) (width 0.5) (layer F.Cu) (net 18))
 (segment (start 151.835 102.195) (end 151.835 100.36) (width 0.5) (layer F.Cu) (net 18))
 (segment (start 120.385 91.195) (end 120.46 91.12) (width 0.5) (layer F.Cu) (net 2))
 (segment (start 110.835 91.195) (end 120.385 91.195) (width 0.5) (layer F.Cu) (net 2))
 (segment (start 118.835 116.695) (end 131.835 116.695) (width 0.5) (layer F.Cu) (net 25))
 (segment (start 131.835 116.695) (end 145.335 116.695) (width 0.5) (layer F.Cu) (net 25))
 (segment (start 145.335 116.695) (end 146.835 116.695) (width 0.5) (layer F.Cu) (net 25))
 (segment (start 149.67 113.86) (end 149.67 108.355) (width 0.5) (layer F.Cu) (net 25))
 (segment (start 146.835 116.695) (end 149.67 113.86) (width 0.5) (layer F.Cu) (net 25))
 (segment (start 110.735 100.195) (end 110.735 96.795) (width 0.5) (layer F.Cu) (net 21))
 (segment (start 110.735 96.795) (end 114.335 93.195) (width 0.5) (layer F.Cu) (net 21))
 (segment (start 127.91 93.195) (end 129.985 91.12) (width 0.5) (layer F.Cu) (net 21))
 (segment (start 114.335 93.195) (end 127.91 93.195) (width 0.5) (layer F.Cu) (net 21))
 (segment (start 110.735 108.595) (end 113.335 111.195) (width 0.5) (layer F.Cu) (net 21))
 (segment (start 110.735 100.195) (end 110.735 108.595) (width 0.5) (layer F.Cu) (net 21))
 (segment (start 110.835 88.695) (end 109.835 88.695) (width 0.5) (layer F.Cu) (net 1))
 (segment (start 108.735 89.795) (end 108.735 100.195) (width 0.5) (layer F.Cu) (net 1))
 (segment (start 109.835 88.695) (end 108.735 89.795) (width 0.5) (layer F.Cu) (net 1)))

